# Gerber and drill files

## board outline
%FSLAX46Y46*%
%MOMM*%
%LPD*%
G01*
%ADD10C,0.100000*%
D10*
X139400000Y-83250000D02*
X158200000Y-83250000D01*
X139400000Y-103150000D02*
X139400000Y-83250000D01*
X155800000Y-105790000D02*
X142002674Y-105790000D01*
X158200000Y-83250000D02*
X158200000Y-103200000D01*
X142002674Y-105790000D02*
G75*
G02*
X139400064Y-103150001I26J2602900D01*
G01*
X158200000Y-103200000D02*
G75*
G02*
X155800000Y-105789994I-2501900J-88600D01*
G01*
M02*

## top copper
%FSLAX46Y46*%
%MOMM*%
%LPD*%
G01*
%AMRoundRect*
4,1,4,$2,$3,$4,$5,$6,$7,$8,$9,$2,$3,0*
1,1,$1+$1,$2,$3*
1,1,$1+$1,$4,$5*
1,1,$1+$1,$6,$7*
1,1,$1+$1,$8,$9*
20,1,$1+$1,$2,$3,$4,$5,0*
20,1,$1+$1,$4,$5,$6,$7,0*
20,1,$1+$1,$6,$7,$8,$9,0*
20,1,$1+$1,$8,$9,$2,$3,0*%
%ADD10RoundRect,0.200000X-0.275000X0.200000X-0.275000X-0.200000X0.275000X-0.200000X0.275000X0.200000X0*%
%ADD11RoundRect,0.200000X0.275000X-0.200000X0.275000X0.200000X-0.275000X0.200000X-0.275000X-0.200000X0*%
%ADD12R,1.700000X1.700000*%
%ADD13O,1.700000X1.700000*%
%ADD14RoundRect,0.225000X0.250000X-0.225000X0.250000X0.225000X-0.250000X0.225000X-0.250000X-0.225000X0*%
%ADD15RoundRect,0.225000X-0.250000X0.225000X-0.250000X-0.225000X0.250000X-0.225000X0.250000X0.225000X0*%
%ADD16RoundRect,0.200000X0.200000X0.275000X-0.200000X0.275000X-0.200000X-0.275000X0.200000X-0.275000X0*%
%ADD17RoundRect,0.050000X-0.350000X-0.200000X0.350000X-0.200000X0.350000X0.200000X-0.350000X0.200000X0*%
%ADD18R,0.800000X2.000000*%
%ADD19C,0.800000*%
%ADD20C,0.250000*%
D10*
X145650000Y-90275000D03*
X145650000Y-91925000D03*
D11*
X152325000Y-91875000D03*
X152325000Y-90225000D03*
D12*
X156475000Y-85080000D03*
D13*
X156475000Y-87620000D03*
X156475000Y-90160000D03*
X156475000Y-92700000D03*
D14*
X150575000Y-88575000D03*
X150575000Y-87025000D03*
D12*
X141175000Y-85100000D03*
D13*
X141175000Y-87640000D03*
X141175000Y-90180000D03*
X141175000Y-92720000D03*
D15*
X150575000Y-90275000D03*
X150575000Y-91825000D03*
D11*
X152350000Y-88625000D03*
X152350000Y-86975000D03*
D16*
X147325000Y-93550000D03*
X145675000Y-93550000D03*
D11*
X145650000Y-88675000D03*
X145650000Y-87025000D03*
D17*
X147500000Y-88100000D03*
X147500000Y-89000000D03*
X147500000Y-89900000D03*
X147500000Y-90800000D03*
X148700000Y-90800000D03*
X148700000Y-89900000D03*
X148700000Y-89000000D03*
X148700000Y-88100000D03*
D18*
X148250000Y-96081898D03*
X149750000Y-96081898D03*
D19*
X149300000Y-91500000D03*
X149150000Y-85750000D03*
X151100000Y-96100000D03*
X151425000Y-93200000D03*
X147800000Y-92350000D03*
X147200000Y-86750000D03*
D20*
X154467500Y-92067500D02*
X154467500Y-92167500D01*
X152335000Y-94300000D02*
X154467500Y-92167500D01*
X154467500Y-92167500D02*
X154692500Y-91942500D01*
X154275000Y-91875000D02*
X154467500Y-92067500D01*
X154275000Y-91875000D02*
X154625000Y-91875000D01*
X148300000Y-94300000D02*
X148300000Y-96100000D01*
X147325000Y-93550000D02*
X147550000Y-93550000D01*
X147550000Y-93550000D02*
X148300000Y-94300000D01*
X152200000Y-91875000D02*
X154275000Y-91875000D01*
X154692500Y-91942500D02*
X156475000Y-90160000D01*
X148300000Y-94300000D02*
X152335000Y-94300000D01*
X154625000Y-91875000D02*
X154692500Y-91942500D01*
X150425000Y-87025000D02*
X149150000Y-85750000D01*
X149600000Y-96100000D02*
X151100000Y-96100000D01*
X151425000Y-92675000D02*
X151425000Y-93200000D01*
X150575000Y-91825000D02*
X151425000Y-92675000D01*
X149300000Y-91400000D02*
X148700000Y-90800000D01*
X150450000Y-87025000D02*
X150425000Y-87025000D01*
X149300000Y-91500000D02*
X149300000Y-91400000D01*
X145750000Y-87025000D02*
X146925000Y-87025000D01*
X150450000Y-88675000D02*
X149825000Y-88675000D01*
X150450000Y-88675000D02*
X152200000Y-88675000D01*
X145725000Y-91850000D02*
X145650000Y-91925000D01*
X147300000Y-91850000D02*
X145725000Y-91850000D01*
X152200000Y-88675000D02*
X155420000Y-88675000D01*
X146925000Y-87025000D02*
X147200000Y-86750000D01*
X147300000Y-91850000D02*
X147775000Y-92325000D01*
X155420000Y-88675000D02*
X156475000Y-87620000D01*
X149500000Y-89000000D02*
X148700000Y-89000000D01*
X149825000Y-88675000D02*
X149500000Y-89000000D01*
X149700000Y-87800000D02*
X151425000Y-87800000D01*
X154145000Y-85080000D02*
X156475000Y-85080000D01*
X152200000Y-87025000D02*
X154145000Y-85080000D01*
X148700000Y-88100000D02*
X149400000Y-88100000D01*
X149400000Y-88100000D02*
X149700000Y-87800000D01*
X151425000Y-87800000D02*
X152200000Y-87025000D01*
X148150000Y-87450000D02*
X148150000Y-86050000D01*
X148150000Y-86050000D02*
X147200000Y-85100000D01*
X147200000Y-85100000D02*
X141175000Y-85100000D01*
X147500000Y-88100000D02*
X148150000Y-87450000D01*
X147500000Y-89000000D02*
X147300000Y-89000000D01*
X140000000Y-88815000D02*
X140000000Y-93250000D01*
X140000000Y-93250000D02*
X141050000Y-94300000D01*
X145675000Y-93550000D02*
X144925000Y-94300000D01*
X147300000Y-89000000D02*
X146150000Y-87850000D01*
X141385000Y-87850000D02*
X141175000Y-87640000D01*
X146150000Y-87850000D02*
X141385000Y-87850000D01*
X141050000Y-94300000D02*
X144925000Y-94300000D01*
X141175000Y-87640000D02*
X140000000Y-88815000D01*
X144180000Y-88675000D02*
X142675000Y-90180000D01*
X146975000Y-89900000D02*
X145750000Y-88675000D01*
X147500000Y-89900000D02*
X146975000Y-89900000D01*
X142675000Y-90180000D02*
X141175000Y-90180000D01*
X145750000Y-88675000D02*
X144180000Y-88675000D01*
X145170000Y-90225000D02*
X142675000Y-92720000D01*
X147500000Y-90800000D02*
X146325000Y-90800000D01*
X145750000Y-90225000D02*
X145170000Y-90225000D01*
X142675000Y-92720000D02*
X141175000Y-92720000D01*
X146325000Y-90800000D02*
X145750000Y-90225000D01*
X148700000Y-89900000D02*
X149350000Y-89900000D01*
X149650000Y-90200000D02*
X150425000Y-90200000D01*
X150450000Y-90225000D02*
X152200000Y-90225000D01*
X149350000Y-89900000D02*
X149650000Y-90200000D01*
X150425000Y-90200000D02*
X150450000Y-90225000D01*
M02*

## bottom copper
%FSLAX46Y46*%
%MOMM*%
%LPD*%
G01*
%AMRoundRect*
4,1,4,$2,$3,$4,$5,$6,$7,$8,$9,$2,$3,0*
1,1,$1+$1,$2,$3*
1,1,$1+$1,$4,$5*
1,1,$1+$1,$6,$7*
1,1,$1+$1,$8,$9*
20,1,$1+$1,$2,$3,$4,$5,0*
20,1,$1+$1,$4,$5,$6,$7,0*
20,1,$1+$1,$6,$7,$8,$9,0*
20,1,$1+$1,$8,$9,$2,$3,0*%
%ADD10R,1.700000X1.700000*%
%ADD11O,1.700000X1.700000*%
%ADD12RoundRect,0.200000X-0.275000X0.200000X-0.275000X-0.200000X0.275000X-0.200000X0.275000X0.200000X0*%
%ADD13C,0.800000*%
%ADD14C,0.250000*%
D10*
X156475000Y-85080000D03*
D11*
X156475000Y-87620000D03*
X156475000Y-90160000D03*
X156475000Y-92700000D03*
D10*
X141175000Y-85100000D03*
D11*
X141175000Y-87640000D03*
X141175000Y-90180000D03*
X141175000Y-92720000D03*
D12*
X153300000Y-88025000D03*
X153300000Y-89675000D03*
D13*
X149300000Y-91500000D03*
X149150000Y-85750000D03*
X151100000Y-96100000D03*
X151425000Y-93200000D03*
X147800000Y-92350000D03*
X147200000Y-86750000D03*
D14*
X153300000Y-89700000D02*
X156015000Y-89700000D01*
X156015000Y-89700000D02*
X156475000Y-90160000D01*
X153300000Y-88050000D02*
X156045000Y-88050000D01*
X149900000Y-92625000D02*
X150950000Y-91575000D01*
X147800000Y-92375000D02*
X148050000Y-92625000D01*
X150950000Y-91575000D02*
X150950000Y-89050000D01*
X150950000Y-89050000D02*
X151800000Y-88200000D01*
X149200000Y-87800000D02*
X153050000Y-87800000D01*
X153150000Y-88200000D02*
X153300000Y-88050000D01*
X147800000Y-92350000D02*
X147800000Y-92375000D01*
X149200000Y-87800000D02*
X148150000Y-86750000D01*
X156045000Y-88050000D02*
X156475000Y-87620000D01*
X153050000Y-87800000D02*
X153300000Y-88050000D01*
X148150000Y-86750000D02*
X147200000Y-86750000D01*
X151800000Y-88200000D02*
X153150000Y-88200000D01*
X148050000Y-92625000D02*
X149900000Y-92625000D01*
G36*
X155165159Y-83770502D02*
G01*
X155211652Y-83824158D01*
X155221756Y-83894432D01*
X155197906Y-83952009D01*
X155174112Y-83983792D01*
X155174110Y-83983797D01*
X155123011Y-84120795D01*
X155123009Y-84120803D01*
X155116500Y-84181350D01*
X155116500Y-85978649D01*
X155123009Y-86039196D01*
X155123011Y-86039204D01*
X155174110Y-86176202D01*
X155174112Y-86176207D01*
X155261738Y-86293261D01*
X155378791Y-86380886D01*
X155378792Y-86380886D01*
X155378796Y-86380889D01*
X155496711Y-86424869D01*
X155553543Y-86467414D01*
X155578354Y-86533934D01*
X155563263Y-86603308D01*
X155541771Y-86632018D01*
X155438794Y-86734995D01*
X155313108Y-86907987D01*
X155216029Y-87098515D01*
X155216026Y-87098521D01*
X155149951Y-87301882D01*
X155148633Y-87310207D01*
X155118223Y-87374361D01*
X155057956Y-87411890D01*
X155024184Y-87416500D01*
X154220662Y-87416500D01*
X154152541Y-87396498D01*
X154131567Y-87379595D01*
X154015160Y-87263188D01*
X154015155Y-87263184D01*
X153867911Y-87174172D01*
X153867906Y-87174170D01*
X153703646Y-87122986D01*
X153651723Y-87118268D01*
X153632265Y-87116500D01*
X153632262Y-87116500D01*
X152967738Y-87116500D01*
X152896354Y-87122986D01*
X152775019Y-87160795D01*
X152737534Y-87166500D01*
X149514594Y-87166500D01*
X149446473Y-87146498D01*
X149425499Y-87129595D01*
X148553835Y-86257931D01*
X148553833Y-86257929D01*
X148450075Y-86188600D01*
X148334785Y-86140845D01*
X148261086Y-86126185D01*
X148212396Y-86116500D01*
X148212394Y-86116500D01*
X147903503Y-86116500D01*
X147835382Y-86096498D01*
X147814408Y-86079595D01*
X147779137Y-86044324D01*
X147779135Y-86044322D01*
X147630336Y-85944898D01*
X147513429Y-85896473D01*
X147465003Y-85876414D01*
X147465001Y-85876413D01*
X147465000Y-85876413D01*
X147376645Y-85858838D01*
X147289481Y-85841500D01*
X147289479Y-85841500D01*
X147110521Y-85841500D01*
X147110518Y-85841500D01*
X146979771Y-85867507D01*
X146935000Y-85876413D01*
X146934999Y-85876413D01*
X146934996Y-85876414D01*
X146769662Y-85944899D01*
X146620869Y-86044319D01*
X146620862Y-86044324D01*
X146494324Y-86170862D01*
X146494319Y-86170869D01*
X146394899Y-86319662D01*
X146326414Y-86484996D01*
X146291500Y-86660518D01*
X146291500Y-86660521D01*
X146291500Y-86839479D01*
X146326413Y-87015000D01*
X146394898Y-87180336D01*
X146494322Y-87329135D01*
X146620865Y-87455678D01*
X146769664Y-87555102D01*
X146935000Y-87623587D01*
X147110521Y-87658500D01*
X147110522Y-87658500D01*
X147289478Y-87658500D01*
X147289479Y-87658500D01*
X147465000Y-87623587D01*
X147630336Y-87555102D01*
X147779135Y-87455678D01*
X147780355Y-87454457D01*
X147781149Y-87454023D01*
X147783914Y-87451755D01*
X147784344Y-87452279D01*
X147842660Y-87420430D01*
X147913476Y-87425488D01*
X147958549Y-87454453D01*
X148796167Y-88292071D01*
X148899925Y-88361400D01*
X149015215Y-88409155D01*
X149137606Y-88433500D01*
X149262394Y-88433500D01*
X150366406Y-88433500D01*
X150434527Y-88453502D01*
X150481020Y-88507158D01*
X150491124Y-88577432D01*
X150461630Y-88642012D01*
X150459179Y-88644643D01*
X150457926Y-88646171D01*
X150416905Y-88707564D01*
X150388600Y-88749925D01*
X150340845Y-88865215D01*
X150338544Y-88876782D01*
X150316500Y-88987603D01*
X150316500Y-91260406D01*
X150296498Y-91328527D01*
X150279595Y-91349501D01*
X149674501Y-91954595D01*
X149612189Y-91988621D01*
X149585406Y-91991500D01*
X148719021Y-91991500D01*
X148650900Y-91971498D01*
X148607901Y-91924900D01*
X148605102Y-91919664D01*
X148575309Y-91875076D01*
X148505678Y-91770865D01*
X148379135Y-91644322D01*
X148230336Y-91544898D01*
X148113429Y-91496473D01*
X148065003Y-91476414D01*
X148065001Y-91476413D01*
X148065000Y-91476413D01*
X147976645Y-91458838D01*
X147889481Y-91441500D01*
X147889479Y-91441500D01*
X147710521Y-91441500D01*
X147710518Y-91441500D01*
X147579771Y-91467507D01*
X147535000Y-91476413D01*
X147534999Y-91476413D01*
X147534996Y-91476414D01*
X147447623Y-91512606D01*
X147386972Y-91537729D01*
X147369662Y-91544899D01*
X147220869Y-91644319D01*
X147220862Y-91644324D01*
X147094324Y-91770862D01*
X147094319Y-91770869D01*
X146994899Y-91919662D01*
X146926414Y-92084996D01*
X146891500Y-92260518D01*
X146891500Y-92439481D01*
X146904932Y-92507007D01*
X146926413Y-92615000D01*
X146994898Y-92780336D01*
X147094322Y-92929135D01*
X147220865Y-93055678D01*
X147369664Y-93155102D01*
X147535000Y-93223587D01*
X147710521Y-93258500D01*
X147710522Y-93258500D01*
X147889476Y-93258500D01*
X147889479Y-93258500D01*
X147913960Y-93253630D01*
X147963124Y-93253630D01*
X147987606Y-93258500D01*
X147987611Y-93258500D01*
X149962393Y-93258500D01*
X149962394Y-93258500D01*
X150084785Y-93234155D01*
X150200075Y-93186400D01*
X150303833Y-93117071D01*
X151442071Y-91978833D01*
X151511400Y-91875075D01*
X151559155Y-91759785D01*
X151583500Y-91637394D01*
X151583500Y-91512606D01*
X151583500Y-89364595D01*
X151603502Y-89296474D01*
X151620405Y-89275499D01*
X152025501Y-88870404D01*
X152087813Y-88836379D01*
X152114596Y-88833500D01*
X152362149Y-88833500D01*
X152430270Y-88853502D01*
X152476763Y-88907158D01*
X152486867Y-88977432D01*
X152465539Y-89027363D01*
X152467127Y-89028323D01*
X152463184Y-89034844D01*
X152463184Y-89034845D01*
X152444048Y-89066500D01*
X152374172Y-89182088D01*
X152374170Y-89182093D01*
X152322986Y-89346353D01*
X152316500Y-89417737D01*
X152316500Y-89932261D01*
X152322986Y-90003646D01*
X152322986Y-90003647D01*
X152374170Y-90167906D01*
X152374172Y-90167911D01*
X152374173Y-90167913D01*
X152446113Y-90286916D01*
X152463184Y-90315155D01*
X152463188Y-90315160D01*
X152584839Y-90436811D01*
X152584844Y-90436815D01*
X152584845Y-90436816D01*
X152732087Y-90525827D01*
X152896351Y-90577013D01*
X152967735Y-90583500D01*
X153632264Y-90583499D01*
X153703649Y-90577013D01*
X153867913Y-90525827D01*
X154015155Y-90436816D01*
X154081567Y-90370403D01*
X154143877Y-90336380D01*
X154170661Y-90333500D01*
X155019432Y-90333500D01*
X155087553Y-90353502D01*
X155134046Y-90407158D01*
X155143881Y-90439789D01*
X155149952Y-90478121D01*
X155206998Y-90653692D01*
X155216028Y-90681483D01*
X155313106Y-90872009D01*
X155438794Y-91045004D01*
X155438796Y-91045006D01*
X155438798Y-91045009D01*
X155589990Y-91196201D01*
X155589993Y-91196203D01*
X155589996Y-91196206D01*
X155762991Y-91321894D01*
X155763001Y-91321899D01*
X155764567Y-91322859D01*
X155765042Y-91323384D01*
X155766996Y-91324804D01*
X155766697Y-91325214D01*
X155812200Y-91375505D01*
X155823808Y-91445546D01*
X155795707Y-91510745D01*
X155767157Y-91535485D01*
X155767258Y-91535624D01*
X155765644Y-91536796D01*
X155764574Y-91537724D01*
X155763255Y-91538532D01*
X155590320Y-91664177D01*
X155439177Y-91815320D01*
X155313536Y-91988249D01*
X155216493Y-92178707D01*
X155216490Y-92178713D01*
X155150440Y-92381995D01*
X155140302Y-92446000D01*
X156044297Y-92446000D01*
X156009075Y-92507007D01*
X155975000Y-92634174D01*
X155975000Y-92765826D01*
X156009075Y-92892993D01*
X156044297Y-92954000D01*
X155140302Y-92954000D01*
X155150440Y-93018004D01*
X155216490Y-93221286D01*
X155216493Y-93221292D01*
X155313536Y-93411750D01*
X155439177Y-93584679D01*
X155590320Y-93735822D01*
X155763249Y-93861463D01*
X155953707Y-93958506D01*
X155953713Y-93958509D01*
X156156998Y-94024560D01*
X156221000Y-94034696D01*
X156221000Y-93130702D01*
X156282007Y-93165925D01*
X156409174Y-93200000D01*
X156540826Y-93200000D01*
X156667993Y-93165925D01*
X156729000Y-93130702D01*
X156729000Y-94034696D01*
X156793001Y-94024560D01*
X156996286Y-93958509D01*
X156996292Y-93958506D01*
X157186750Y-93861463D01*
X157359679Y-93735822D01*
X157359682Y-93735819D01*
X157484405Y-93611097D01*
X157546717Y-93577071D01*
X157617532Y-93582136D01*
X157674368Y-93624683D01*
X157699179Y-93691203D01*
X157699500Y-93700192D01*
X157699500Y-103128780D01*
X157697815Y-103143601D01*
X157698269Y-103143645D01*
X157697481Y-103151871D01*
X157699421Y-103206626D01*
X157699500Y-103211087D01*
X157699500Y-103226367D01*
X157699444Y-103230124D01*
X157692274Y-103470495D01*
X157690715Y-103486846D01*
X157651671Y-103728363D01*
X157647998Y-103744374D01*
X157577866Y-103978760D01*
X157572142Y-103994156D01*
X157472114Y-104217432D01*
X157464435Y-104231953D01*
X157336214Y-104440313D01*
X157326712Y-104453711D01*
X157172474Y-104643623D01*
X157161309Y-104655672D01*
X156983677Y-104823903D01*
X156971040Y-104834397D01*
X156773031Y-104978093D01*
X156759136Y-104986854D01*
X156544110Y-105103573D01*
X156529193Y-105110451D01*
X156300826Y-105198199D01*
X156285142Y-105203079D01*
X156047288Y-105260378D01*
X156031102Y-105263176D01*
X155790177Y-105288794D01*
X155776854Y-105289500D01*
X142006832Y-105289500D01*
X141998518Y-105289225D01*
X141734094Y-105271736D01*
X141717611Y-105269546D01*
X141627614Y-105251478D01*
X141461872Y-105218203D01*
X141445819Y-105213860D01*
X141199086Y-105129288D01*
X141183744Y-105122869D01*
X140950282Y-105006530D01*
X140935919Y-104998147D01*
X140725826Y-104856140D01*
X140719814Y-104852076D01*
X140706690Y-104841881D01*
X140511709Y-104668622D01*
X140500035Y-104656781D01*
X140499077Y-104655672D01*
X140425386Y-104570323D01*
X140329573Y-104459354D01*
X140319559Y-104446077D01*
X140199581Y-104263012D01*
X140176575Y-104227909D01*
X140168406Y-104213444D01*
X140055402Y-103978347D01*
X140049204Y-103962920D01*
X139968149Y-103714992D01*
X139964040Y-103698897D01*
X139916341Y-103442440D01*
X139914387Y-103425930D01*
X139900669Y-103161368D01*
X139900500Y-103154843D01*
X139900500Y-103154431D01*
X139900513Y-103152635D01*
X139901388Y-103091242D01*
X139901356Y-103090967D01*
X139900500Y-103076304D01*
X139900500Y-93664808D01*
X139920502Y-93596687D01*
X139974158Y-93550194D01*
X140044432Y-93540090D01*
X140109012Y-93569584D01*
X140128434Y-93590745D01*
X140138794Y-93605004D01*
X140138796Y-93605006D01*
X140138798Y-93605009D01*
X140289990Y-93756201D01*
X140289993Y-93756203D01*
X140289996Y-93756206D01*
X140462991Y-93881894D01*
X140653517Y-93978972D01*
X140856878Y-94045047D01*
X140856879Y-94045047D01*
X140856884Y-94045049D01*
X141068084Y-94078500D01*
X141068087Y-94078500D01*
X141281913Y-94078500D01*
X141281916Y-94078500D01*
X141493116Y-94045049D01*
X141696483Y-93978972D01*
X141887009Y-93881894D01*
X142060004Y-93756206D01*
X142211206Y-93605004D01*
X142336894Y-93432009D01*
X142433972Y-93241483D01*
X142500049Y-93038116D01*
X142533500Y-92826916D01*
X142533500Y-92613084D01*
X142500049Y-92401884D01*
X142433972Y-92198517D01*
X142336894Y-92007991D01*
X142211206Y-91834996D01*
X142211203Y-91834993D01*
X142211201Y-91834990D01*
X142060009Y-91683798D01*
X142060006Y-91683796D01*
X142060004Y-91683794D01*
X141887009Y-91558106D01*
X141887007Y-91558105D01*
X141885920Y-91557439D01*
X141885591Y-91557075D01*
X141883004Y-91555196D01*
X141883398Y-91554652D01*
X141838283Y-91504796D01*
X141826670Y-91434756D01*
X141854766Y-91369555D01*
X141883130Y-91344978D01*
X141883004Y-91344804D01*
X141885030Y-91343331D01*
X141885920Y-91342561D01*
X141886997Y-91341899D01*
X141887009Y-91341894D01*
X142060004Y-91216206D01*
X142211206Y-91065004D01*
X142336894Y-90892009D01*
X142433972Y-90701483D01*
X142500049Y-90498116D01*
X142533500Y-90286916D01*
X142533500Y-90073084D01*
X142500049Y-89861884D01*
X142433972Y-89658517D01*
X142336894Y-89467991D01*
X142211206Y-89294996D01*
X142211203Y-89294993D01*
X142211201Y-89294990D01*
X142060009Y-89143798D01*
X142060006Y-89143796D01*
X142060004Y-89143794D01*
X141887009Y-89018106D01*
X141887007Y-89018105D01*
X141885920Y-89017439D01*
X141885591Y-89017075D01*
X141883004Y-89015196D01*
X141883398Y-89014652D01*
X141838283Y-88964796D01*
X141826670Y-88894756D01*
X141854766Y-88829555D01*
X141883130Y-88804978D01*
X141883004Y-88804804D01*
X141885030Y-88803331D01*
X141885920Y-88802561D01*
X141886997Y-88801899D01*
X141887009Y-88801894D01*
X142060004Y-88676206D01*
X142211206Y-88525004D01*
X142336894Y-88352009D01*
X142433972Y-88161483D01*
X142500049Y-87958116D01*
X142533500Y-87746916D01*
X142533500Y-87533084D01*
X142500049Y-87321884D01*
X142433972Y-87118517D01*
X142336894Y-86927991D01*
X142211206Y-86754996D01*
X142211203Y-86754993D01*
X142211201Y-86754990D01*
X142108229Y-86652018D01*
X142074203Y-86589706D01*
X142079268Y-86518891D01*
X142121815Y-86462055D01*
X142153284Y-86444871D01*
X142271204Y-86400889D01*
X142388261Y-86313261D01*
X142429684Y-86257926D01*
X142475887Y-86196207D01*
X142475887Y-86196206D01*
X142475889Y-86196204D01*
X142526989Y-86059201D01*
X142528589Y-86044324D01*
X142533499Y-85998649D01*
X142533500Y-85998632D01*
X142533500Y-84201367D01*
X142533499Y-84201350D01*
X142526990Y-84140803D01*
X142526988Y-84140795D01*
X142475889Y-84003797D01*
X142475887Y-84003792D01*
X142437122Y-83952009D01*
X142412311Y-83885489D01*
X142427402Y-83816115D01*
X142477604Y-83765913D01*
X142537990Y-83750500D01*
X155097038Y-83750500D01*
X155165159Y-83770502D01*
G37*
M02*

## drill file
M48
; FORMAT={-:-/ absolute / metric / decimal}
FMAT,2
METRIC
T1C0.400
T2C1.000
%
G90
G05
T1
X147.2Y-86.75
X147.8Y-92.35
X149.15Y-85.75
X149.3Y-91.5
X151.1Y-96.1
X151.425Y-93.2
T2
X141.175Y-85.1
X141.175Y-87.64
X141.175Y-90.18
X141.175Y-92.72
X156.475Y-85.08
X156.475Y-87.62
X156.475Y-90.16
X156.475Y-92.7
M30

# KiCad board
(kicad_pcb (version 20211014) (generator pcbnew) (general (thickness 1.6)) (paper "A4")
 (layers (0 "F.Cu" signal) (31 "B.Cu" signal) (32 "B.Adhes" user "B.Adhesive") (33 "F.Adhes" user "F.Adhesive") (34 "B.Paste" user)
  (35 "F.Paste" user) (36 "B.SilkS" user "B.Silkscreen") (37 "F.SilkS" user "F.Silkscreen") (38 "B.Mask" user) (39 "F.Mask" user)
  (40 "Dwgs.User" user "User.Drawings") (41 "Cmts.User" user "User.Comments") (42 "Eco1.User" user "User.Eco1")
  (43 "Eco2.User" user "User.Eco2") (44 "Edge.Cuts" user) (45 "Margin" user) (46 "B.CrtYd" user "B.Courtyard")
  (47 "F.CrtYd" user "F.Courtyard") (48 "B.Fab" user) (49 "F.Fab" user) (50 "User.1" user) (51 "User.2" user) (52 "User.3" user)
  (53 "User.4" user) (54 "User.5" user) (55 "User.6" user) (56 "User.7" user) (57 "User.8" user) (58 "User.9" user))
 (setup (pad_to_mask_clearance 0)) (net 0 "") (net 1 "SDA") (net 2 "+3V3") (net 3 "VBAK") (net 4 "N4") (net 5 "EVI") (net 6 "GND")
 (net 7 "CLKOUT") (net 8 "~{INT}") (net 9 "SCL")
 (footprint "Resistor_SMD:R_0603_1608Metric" (layer "F.Cu") (at 145.65 91.1 -90)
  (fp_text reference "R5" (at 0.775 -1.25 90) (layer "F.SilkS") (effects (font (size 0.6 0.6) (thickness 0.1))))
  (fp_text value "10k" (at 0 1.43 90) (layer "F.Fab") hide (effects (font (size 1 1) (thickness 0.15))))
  (pad "1" smd roundrect (at -0.825 0 270) (size 0.8 0.95) (layers "F.Cu" "F.Paste" "F.Mask") (roundrect_rratio 0.25) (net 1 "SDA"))
  (pad "2" smd roundrect (at 0.825 0 270) (size 0.8 0.95) (layers "F.Cu" "F.Paste" "F.Mask") (roundrect_rratio 0.25) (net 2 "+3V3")))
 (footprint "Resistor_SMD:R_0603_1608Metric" (layer "F.Cu") (at 152.325 91.05 90)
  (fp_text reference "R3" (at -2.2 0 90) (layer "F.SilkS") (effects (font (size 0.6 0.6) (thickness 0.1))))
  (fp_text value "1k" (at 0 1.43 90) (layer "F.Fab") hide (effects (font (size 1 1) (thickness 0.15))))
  (pad "1" smd roundrect (at -0.825 0 90) (size 0.8 0.95) (layers "F.Cu" "F.Paste" "F.Mask") (roundrect_rratio 0.25) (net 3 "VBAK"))
  (pad "2" smd roundrect (at 0.825 0 90) (size 0.8 0.95) (layers "F.Cu" "F.Paste" "F.Mask") (roundrect_rratio 0.25) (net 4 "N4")))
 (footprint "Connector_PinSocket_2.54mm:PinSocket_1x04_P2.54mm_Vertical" (layer "F.Cu") (at 156.475 85.08)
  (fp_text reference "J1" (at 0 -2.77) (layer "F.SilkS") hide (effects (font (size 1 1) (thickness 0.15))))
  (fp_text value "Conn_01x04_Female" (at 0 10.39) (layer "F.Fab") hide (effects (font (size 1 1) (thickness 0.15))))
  (pad "1" thru_hole rect (at 0 0) (size 1.7 1.7) (drill 1) (layers *.Cu *.Mask) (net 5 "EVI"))
  (pad "2" thru_hole oval (at 0 2.54) (size 1.7 1.7) (drill 1) (layers *.Cu *.Mask) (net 2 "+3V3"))
  (pad "3" thru_hole oval (at 0 5.08) (size 1.7 1.7) (drill 1) (layers *.Cu *.Mask) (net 3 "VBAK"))
  (pad "4" thru_hole oval (at 0 7.62) (size 1.7 1.7) (drill 1) (layers *.Cu *.Mask) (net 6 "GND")))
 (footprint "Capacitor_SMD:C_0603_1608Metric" (layer "F.Cu") (at 150.575 87.8 90)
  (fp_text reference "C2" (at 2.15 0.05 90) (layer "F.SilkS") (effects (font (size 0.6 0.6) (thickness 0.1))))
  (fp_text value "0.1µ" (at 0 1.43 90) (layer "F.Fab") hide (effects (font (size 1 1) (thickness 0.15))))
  (pad "1" smd roundrect (at -0.775 0 90) (size 0.9 0.95) (layers "F.Cu" "F.Paste" "F.Mask") (roundrect_rratio 0.25) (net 2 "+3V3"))
  (pad "2" smd roundrect (at 0.775 0 90) (size 0.9 0.95) (layers "F.Cu" "F.Paste" "F.Mask") (roundrect_rratio 0.25) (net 6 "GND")))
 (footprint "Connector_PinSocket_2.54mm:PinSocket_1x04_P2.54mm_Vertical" (layer "F.Cu") (at 141.175 85.1)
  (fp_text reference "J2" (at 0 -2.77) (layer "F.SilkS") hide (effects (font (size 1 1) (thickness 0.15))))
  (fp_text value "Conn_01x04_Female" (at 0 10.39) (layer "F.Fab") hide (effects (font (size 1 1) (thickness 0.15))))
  (pad "1" thru_hole rect (at 0 0) (size 1.7 1.7) (drill 1) (layers *.Cu *.Mask) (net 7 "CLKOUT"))
  (pad "2" thru_hole oval (at 0 2.54) (size 1.7 1.7) (drill 1) (layers *.Cu *.Mask) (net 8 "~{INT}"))
  (pad "3" thru_hole oval (at 0 5.08) (size 1.7 1.7) (drill 1) (layers *.Cu *.Mask) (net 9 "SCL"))
  (pad "4" thru_hole oval (at 0 7.62) (size 1.7 1.7) (drill 1) (layers *.Cu *.Mask) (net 1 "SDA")))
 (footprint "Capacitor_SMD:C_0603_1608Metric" (layer "F.Cu") (at 150.575 91.05 -90)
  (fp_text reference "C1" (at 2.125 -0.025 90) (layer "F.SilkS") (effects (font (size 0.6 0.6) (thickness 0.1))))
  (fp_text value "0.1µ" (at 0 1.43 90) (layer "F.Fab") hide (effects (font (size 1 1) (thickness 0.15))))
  (pad "1" smd roundrect (at -0.775 0 270) (size 0.9 0.95) (layers "F.Cu" "F.Paste" "F.Mask") (roundrect_rratio 0.25) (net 4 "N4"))
  (pad "2" smd roundrect (at 0.775 0 270) (size 0.9 0.95) (layers "F.Cu" "F.Paste" "F.Mask") (roundrect_rratio 0.25) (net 6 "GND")))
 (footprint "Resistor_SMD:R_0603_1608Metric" (layer "F.Cu") (at 152.35 87.8 90)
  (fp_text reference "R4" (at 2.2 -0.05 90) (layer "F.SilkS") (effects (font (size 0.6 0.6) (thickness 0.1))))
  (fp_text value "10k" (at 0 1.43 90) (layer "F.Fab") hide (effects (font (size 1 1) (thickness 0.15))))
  (pad "1" smd roundrect (at -0.825 0 90) (size 0.8 0.95) (layers "F.Cu" "F.Paste" "F.Mask") (roundrect_rratio 0.25) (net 2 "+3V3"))
  (pad "2" smd roundrect (at 0.825 0 90) (size 0.8 0.95) (layers "F.Cu" "F.Paste" "F.Mask") (roundrect_rratio 0.25) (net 5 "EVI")))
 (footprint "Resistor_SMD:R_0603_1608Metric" (layer "F.Cu") (at 146.5 93.55 180)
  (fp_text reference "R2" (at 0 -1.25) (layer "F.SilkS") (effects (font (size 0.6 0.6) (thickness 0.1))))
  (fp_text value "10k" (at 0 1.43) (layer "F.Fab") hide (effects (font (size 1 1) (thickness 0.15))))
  (pad "1" smd roundrect (at -0.825 0 180) (size 0.8 0.95) (layers "F.Cu" "F.Paste" "F.Mask") (roundrect_rratio 0.25) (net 3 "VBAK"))
  (pad "2" smd roundrect (at 0.825 0 180) (size 0.8 0.95) (layers "F.Cu" "F.Paste" "F.Mask") (roundrect_rratio 0.25) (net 8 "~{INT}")))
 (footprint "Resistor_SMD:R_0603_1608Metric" (layer "F.Cu") (at 145.65 87.85 90)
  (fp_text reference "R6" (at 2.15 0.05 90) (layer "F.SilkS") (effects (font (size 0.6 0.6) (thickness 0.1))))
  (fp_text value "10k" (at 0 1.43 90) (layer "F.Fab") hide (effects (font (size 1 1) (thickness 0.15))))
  (pad "1" smd roundrect (at -0.825 0 90) (size 0.8 0.95) (layers "F.Cu" "F.Paste" "F.Mask") (roundrect_rratio 0.25) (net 9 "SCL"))
  (pad "2" smd roundrect (at 0.825 0 90) (size 0.8 0.95) (layers "F.Cu" "F.Paste" "F.Mask") (roundrect_rratio 0.25) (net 2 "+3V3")))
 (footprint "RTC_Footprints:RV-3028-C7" (layer "F.Cu") (at 148.1 89.45)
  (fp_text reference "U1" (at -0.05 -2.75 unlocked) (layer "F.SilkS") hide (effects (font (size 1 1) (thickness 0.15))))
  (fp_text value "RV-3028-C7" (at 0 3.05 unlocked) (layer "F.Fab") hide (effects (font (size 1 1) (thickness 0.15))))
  (pad "1" smd roundrect (at -0.6 -1.35) (size 0.8 0.5) (layers "F.Cu" "F.Paste" "F.Mask") (roundrect_rratio 0.1) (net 7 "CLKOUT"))
  (pad "2" smd roundrect (at -0.6 -0.45) (size 0.8 0.5) (layers "F.Cu" "F.Paste" "F.Mask") (roundrect_rratio 0.1) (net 8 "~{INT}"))
  (pad "3" smd roundrect (at -0.6 0.45) (size 0.8 0.5) (layers "F.Cu" "F.Paste" "F.Mask") (roundrect_rratio 0.1) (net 9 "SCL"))
  (pad "4" smd roundrect (at -0.6 1.35) (size 0.8 0.5) (layers "F.Cu" "F.Paste" "F.Mask") (roundrect_rratio 0.1) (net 1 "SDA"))
  (pad "5" smd roundrect (at 0.6 1.35) (size 0.8 0.5) (layers "F.Cu" "F.Paste" "F.Mask") (roundrect_rratio 0.1) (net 6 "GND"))
  (pad "6" smd roundrect (at 0.6 0.45) (size 0.8 0.5) (layers "F.Cu" "F.Paste" "F.Mask") (roundrect_rratio 0.1) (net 4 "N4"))
  (pad "7" smd roundrect (at 0.6 -0.45) (size 0.8 0.5) (layers "F.Cu" "F.Paste" "F.Mask") (roundrect_rratio 0.1) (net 2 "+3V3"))
  (pad "8" smd roundrect (at 0.6 -1.35) (size 0.8 0.5) (layers "F.Cu" "F.Paste" "F.Mask") (roundrect_rratio 0.1) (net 5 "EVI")))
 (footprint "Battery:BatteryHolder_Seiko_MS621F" (layer "F.Cu") (at 149 96.081898 90)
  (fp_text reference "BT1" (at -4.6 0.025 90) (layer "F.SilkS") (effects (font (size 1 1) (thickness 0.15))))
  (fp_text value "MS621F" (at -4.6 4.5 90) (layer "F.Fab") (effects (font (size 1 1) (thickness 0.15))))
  (pad "1" smd rect (at 0 -0.75 90) (size 2 0.8) (layers "F.Cu" "F.Paste" "F.Mask") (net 3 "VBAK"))
  (pad "2" smd rect (at 0 0.75 90) (size 2 0.8) (layers "F.Cu" "F.Paste" "F.Mask") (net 6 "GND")))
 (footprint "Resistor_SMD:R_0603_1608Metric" (layer "B.Cu") (at 153.3 88.85 -90)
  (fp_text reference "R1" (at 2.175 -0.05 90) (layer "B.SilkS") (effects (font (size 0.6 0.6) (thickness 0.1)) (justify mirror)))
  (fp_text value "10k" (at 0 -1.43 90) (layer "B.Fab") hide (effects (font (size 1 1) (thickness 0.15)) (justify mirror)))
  (pad "1" smd roundrect (at -0.825 0 270) (size 0.8 0.95) (layers "B.Cu" "B.Paste" "B.Mask") (roundrect_rratio 0.25) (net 2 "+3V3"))
  (pad "2" smd roundrect (at 0.825 0 270) (size 0.8 0.95) (layers "B.Cu" "B.Paste" "B.Mask") (roundrect_rratio 0.25) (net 3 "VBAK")))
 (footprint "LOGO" (layer "B.Cu") (at 155.1 103.2 180)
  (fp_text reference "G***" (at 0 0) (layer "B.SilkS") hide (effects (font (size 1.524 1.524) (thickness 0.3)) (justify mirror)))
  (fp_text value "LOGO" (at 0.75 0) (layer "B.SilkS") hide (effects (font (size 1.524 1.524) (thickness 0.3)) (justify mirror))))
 (gr_line (start 139.4 83.25) (end 158.2 83.25) (layer "Edge.Cuts") (width 0.1))
 (gr_line (start 139.4 103.15) (end 139.4 83.25) (layer "Edge.Cuts") (width 0.1))
 (gr_line (start 155.8 105.79) (end 142.002674 105.79) (layer "Edge.Cuts") (width 0.1))
 (gr_line (start 158.2 83.25) (end 158.2 103.2) (layer "Edge.Cuts") (width 0.1))
 (gr_arc (start 142.002674 105.79) (mid 140.149063 105.014466) (end 139.4 103.15) (layer "Edge.Cuts") (width 0.1))
 (gr_arc (start 158.2 103.2) (mid 157.534401 104.990198) (end 155.8 105.79) (layer "Edge.Cuts") (width 0.1))
 (segment (start 154.4675 92.0675) (end 154.4675 92.1675) (width 0.25) (layer "F.Cu") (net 3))
 (segment (start 152.335 94.3) (end 154.4675 92.1675) (width 0.25) (layer "F.Cu") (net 3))
 (segment (start 154.4675 92.1675) (end 154.6925 91.9425) (width 0.25) (layer "F.Cu") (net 3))
 (segment (start 154.275 91.875) (end 154.4675 92.0675) (width 0.25) (layer "F.Cu") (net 3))
 (segment (start 154.275 91.875) (end 154.625 91.875) (width 0.25) (layer "F.Cu") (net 3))
 (segment (start 148.3 94.3) (end 148.3 96.1) (width 0.25) (layer "F.Cu") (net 3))
 (segment (start 147.325 93.55) (end 147.55 93.55) (width 0.25) (layer "F.Cu") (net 3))
 (segment (start 147.55 93.55) (end 148.3 94.3) (width 0.25) (layer "F.Cu") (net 3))
 (segment (start 152.2 91.875) (end 154.275 91.875) (width 0.25) (layer "F.Cu") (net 3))
 (segment (start 154.6925 91.9425) (end 156.475 90.16) (width 0.25) (layer "F.Cu") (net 3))
 (segment (start 148.3 94.3) (end 152.335 94.3) (width 0.25) (layer "F.Cu") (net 3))
 (segment (start 154.625 91.875) (end 154.6925 91.9425) (width 0.25) (layer "F.Cu") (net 3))
 (segment (start 153.3 89.7) (end 156.015 89.7) (width 0.25) (layer "B.Cu") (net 3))
 (segment (start 156.015 89.7) (end 156.475 90.16) (width 0.25) (layer "B.Cu") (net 3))
 (segment (start 150.425 87.025) (end 149.15 85.75) (width 0.25) (layer "F.Cu") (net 6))
 (segment (start 149.6 96.1) (end 151.1 96.1) (width 0.25) (layer "F.Cu") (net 6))
 (segment (start 151.425 92.675) (end 151.425 93.2) (width 0.25) (layer "F.Cu") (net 6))
 (segment (start 150.575 91.825) (end 151.425 92.675) (width 0.25) (layer "F.Cu") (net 6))
 (segment (start 149.3 91.4) (end 148.7 90.8) (width 0.25) (layer "F.Cu") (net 6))
 (segment (start 150.45 87.025) (end 150.425 87.025) (width 0.25) (layer "F.Cu") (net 6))
 (segment (start 149.3 91.5) (end 149.3 91.4) (width 0.25) (layer "F.Cu") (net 6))
 (via (at 149.3 91.5) (size 0.8) (drill 0.4) (layers "F.Cu" "B.Cu") (free) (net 6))
 (via (at 149.15 85.75) (size 0.8) (drill 0.4) (layers "F.Cu" "B.Cu") (free) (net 6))
 (via (at 151.1 96.1) (size 0.8) (drill 0.4) (layers "F.Cu" "B.Cu") (free) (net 6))
 (via (at 151.425 93.2) (size 0.8) (drill 0.4) (layers "F.Cu" "B.Cu") (free) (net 6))
 (segment (start 145.75 87.025) (end 146.925 87.025) (width 0.25) (layer "F.Cu") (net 2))
 (segment (start 150.45 88.675) (end 149.825 88.675) (width 0.25) (layer "F.Cu") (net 2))
 (segment (start 150.45 88.675) (end 152.2 88.675) (width 0.25) (layer "F.Cu") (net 2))
 (segment (start 145.725 91.85) (end 145.65 91.925) (width 0.25) (layer "F.Cu") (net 2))
 (segment (start 147.3 91.85) (end 145.725 91.85) (width 0.25) (layer "F.Cu") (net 2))
 (segment (start 152.2 88.675) (end 155.42 88.675) (width 0.25) (layer "F.Cu") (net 2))
 (segment (start 146.925 87.025) (end 147.2 86.75) (width 0.25) (layer "F.Cu") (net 2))
 (segment (start 147.3 91.85) (end 147.775 92.325) (width 0.25) (layer "F.Cu") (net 2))
 (segment (start 155.42 88.675) (end 156.475 87.62) (width 0.25) (layer "F.Cu") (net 2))
 (segment (start 149.5 89) (end 148.7 89) (width 0.25) (layer "F.Cu") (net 2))
 (segment (start 149.825 88.675) (end 149.5 89) (width 0.25) (layer "F.Cu") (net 2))
 (via (at 147.8 92.35) (size 0.8) (drill 0.4) (layers "F.Cu" "B.Cu") (free) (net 2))
 (via (at 147.2 86.75) (size 0.8) (drill 0.4) (layers "F.Cu" "B.Cu") (free) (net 2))
 (segment (start 153.3 88.05) (end 156.045 88.05) (width 0.25) (layer "B.Cu") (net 2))
 (segment (start 149.9 92.625) (end 150.95 91.575) (width 0.25) (layer "B.Cu") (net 2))
 (segment (start 147.8 92.375) (end 148.05 92.625) (width 0.25) (layer "B.Cu") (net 2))
 (segment (start 150.95 91.575) (end 150.95 89.05) (width 0.25) (layer "B.Cu") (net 2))
 (segment (start 150.95 89.05) (end 151.8 88.2) (width 0.25) (layer "B.Cu") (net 2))
 (segment (start 149.2 87.8) (end 153.05 87.8) (width 0.25) (layer "B.Cu") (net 2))
 (segment (start 153.15 88.2) (end 153.3 88.05) (width 0.25) (layer "B.Cu") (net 2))
 (segment (start 147.8 92.35) (end 147.8 92.375) (width 0.25) (layer "B.Cu") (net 2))
 (segment (start 149.2 87.8) (end 148.15 86.75) (width 0.25) (layer "B.Cu") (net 2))
 (segment (start 156.045 88.05) (end 156.475 87.62) (width 0.25) (layer "B.Cu") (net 2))
 (segment (start 153.05 87.8) (end 153.3 88.05) (width 0.25) (layer "B.Cu") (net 2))
 (segment (start 148.15 86.75) (end 147.2 86.75) (width 0.25) (layer "B.Cu") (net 2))
 (segment (start 151.8 88.2) (end 153.15 88.2) (width 0.25) (layer "B.Cu") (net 2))
 (segment (start 148.05 92.625) (end 149.9 92.625) (width 0.25) (layer "B.Cu") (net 2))
 (segment (start 149.7 87.8) (end 151.425 87.8) (width 0.25) (layer "F.Cu") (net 5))
 (segment (start 154.145 85.08) (end 156.475 85.08) (width 0.25) (layer "F.Cu") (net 5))
 (segment (start 152.2 87.025) (end 154.145 85.08) (width 0.25) (layer "F.Cu") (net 5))
 (segment (start 148.7 88.1) (end 149.4 88.1) (width 0.25) (layer "F.Cu") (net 5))
 (segment (start 149.4 88.1) (end 149.7 87.8) (width 0.25) (layer "F.Cu") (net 5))
 (segment (start 151.425 87.8) (end 152.2 87.025) (width 0.25) (layer "F.Cu") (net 5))
 (segment (start 148.15 87.45) (end 148.15 86.05) (width 0.25) (layer "F.Cu") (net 7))
 (segment (start 148.15 86.05) (end 147.2 85.1) (width 0.25) (layer "F.Cu") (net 7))
 (segment (start 147.2 85.1) (end 141.175 85.1) (width 0.25) (layer "F.Cu") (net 7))
 (segment (start 147.5 88.1) (end 148.15 87.45) (width 0.25) (layer "F.Cu") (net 7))
 (segment (start 147.5 89) (end 147.3 89) (width 0.25) (layer "F.Cu") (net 8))
 (segment (start 140 88.815) (end 140 93.25) (width 0.25) (layer "F.Cu") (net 8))
 (segment (start 140 93.25) (end 141.05 94.3) (width 0.25) (layer "F.Cu") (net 8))
 (segment (start 145.675 93.55) (end 144.925 94.3) (width 0.25) (layer "F.Cu") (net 8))
 (segment (start 147.3 89) (end 146.15 87.85) (width 0.25) (layer "F.Cu") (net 8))
 (segment (start 141.385 87.85) (end 141.175 87.64) (width 0.25) (layer "F.Cu") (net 8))
 (segment (start 146.15 87.85) (end 141.385 87.85) (width 0.25) (layer "F.Cu") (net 8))
 (segment (start 141.05 94.3) (end 144.925 94.3) (width 0.25) (layer "F.Cu") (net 8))
 (segment (start 141.175 87.64) (end 140 88.815) (width 0.25) (layer "F.Cu") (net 8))
 (segment (start 144.18 88.675) (end 142.675 90.18) (width 0.25) (layer "F.Cu") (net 9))
 (segment (start 146.975 89.9) (end 145.75 88.675) (width 0.25) (layer "F.Cu") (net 9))
 (segment (start 147.5 89.9) (end 146.975 89.9) (width 0.25) (layer "F.Cu") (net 9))
 (segment (start 142.675 90.18) (end 141.175 90.18) (width 0.25) (layer "F.Cu") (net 9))
 (segment (start 145.75 88.675) (end 144.18 88.675) (width 0.25) (layer "F.Cu") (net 9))
 (segment (start 145.17 90.225) (end 142.675 92.72) (width 0.25) (layer "F.Cu") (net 1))
 (segment (start 147.5 90.8) (end 146.325 90.8) (width 0.25) (layer "F.Cu") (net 1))
 (segment (start 145.75 90.225) (end 145.17 90.225) (width 0.25) (layer "F.Cu") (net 1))
 (segment (start 142.675 92.72) (end 141.175 92.72) (width 0.25) (layer "F.Cu") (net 1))
 (segment (start 146.325 90.8) (end 145.75 90.225) (width 0.25) (layer "F.Cu") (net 1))
 (segment (start 148.7 89.9) (end 149.35 89.9) (width 0.25) (layer "F.Cu") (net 4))
 (segment (start 149.65 90.2) (end 150.425 90.2) (width 0.25) (layer "F.Cu") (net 4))
 (segment (start 150.45 90.225) (end 152.2 90.225) (width 0.25) (layer "F.Cu") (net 4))
 (segment (start 149.35 89.9) (end 149.65 90.2) (width 0.25) (layer "F.Cu") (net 4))
 (segment (start 150.425 90.2) (end 150.45 90.225) (width 0.25) (layer "F.Cu") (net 4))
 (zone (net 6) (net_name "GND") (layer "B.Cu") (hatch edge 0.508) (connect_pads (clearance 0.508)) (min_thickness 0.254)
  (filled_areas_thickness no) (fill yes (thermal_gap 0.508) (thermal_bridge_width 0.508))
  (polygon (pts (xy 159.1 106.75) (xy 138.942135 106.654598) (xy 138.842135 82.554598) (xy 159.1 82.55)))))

